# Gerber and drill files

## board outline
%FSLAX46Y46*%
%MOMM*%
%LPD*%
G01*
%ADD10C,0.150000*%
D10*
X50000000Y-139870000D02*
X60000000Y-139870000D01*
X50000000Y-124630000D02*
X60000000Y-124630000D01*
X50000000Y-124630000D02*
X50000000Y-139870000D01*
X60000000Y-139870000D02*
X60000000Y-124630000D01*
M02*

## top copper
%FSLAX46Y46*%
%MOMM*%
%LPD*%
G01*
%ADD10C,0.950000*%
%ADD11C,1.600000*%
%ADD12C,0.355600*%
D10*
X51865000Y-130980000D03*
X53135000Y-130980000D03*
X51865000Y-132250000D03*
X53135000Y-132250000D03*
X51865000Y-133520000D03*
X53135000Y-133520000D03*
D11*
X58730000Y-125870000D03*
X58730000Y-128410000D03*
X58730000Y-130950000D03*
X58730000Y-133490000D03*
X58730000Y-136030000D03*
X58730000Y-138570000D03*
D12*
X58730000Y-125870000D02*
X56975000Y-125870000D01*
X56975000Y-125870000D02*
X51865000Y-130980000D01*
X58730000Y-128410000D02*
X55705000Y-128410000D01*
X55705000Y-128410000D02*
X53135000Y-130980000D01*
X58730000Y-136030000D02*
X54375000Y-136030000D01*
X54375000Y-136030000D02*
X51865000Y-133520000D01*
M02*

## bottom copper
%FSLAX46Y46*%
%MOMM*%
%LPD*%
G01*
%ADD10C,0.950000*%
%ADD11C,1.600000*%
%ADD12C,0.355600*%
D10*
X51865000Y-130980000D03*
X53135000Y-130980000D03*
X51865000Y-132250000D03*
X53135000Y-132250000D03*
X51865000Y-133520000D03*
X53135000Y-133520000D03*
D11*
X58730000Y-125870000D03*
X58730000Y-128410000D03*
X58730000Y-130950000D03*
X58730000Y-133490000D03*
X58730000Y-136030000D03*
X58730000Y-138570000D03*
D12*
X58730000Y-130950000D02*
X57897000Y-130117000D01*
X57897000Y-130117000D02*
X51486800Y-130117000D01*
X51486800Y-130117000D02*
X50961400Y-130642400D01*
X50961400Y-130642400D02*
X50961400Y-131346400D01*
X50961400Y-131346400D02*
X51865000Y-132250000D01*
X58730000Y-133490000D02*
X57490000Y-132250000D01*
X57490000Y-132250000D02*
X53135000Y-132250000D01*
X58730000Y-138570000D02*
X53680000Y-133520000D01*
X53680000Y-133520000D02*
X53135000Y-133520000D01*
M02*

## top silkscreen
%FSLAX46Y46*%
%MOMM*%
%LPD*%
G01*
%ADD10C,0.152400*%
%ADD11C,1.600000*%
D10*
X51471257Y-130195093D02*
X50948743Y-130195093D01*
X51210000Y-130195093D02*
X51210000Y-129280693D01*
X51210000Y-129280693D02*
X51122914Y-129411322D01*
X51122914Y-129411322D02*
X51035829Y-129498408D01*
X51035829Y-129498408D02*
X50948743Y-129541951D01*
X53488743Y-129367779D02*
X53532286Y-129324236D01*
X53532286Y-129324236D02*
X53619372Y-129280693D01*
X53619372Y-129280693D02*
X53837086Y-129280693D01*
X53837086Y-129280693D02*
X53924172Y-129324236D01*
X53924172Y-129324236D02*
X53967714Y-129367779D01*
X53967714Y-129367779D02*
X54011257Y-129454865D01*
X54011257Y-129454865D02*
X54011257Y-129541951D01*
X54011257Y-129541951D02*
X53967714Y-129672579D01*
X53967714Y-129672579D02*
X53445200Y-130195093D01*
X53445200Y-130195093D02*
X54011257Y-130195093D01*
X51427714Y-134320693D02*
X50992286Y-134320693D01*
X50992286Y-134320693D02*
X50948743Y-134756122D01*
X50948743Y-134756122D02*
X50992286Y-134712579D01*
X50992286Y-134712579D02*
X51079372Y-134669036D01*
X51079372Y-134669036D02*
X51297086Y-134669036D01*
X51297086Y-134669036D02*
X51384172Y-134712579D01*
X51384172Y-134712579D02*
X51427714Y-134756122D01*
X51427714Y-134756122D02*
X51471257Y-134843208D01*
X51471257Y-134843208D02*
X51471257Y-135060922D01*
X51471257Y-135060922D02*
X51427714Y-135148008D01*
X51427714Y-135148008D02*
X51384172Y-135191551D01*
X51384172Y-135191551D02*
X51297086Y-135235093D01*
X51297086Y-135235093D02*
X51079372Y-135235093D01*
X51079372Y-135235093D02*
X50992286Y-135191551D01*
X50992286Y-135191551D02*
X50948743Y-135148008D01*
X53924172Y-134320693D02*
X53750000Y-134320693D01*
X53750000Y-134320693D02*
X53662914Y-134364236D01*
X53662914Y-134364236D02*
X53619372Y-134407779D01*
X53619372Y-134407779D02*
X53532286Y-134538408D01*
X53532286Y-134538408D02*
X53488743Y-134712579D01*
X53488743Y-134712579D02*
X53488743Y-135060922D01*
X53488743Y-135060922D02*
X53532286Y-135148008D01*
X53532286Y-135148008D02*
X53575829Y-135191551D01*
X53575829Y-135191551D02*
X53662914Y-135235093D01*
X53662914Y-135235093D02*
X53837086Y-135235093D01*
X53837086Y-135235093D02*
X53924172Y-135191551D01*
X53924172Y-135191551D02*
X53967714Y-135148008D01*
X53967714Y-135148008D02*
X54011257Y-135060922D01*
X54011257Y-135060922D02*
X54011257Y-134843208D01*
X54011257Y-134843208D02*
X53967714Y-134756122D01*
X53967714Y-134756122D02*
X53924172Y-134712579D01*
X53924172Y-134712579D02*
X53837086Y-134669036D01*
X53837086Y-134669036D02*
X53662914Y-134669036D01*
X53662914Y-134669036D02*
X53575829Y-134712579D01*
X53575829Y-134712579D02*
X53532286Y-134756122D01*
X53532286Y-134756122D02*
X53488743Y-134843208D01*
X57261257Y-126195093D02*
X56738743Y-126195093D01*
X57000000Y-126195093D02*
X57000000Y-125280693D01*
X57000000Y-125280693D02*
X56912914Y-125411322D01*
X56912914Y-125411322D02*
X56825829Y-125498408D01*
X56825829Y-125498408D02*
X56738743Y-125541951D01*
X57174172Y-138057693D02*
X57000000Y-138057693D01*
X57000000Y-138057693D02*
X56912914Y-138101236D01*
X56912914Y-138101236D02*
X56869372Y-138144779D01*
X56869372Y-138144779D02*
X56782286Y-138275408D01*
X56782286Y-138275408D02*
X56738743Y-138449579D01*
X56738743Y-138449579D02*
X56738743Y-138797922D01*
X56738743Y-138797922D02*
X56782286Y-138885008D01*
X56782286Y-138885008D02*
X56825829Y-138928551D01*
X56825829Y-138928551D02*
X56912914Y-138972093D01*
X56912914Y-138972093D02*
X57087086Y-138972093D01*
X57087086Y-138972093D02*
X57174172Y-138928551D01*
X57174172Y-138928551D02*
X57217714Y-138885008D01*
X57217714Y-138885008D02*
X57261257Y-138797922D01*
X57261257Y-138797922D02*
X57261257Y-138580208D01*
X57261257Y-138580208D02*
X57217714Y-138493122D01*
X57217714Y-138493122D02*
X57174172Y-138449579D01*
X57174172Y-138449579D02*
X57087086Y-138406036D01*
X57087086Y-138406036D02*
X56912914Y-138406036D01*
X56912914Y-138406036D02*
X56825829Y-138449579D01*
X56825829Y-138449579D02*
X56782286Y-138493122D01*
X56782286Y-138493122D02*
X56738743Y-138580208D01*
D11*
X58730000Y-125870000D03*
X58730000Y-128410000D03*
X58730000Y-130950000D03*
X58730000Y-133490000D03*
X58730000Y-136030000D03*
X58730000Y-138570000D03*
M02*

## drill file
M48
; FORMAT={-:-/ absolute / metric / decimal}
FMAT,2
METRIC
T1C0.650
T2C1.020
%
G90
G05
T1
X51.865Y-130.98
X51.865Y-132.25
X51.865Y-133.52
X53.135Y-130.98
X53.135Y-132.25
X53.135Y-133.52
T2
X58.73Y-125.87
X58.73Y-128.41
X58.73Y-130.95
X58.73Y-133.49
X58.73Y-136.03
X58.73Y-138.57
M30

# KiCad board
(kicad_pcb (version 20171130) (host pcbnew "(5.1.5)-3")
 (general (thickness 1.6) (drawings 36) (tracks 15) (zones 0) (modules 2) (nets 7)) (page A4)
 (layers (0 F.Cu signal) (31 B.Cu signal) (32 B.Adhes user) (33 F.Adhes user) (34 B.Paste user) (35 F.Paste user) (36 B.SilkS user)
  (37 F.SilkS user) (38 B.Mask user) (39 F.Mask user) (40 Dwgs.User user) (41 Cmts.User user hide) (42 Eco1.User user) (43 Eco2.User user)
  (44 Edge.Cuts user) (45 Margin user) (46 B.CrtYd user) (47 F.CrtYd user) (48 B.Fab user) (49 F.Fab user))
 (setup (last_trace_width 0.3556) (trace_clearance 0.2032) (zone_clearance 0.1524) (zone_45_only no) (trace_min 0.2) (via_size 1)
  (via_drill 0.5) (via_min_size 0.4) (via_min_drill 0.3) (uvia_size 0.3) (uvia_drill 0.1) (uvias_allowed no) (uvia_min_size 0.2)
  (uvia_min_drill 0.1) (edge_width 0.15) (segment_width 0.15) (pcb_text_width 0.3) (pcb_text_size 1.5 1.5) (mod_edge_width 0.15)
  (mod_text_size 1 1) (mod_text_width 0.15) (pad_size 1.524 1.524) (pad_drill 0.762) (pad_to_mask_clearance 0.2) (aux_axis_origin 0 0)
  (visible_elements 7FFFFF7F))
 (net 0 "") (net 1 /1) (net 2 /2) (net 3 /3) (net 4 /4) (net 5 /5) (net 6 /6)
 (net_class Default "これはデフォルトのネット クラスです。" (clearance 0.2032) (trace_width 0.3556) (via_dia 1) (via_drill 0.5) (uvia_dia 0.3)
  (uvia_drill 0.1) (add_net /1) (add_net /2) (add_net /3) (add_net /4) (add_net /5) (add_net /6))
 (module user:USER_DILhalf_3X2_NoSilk (layer F.Cu) (at 52.5 132.25)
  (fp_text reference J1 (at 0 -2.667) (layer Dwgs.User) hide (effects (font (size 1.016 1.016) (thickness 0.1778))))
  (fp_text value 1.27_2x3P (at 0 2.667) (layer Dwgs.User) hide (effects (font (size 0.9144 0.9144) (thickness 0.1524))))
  (pad 1 thru_hole circle (at -0.635 -1.27) (size 0.95 0.95) (drill 0.65) (layers *.Cu *.Mask) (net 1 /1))
  (pad 2 thru_hole circle (at 0.635 -1.27) (size 0.95 0.95) (drill 0.65) (layers *.Cu *.Mask) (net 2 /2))
  (pad 3 thru_hole circle (at -0.635 0) (size 0.95 0.95) (drill 0.65) (layers *.Cu *.Mask) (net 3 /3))
  (pad 4 thru_hole circle (at 0.635 0) (size 0.95 0.95) (drill 0.65) (layers *.Cu *.Mask) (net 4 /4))
  (pad 5 thru_hole circle (at -0.635 1.27) (size 0.95 0.95) (drill 0.65) (layers *.Cu *.Mask) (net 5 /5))
  (pad 6 thru_hole circle (at 0.635 1.27) (size 0.95 0.95) (drill 0.65) (layers *.Cu *.Mask) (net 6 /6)))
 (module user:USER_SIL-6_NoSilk (layer F.Cu) (at 58.73 132.22 270)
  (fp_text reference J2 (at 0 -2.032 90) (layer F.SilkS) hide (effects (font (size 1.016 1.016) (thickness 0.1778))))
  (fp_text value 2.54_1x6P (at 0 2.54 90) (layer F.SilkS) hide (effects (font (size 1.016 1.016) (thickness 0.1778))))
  (pad 1 thru_hole circle (at -6.35 0 270) (size 1.6 1.6) (drill 1.02) (layers *.Cu *.Mask F.SilkS) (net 1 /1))
  (pad 2 thru_hole circle (at -3.81 0 270) (size 1.6 1.6) (drill 1.02) (layers *.Cu *.Mask F.SilkS) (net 2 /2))
  (pad 3 thru_hole circle (at -1.27 0 270) (size 1.6 1.6) (drill 1.02) (layers *.Cu *.Mask F.SilkS) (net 3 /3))
  (pad 4 thru_hole circle (at 1.27 0 270) (size 1.6 1.6) (drill 1.02) (layers *.Cu *.Mask F.SilkS) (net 4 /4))
  (pad 5 thru_hole circle (at 3.81 0 270) (size 1.6 1.6) (drill 1.02) (layers *.Cu *.Mask F.SilkS) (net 5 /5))
  (pad 6 thru_hole circle (at 6.35 0 270) (size 1.6 1.6) (drill 1.02) (layers *.Cu *.Mask F.SilkS) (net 6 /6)))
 (gr_line (start 50 139.87) (end 60 139.87) (angle 90) (layer Edge.Cuts) (width 0.15))
 (gr_line (start 50 124.63) (end 60 124.63) (angle 90) (layer Edge.Cuts) (width 0.15))
 (gr_line (start 50 124.63) (end 50 139.87) (angle 90) (layer Edge.Cuts) (width 0.15))
 (gr_line (start 60 139.87) (end 60 124.63) (angle 90) (layer Edge.Cuts) (width 0.15))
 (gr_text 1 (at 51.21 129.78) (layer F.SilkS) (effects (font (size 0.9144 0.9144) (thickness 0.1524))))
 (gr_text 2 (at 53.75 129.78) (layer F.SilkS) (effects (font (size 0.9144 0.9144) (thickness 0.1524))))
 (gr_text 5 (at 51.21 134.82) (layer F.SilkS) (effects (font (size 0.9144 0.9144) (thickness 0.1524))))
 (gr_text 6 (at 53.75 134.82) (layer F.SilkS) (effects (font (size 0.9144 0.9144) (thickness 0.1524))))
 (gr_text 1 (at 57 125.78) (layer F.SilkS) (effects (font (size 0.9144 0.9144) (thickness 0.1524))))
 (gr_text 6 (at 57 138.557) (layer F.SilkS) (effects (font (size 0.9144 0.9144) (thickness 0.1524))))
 (segment (start 58.73 125.87) (end 56.975 125.87) (width 0.3556) (layer F.Cu) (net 1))
 (segment (start 56.975 125.87) (end 51.865 130.98) (width 0.3556) (layer F.Cu) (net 1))
 (segment (start 58.73 128.41) (end 55.705 128.41) (width 0.3556) (layer F.Cu) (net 2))
 (segment (start 55.705 128.41) (end 53.135 130.98) (width 0.3556) (layer F.Cu) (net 2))
 (segment (start 58.73 130.95) (end 57.897 130.117) (width 0.3556) (layer B.Cu) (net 3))
 (segment (start 57.897 130.117) (end 51.4868 130.117) (width 0.3556) (layer B.Cu) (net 3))
 (segment (start 51.4868 130.117) (end 50.9614 130.6424) (width 0.3556) (layer B.Cu) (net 3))
 (segment (start 50.9614 130.6424) (end 50.9614 131.3464) (width 0.3556) (layer B.Cu) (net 3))
 (segment (start 50.9614 131.3464) (end 51.865 132.25) (width 0.3556) (layer B.Cu) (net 3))
 (segment (start 58.73 133.49) (end 57.49 132.25) (width 0.3556) (layer B.Cu) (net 4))
 (segment (start 57.49 132.25) (end 53.135 132.25) (width 0.3556) (layer B.Cu) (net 4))
 (segment (start 58.73 136.03) (end 54.375 136.03) (width 0.3556) (layer F.Cu) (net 5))
 (segment (start 54.375 136.03) (end 51.865 133.52) (width 0.3556) (layer F.Cu) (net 5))
 (segment (start 58.73 138.57) (end 53.68 133.52) (width 0.3556) (layer B.Cu) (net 6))
 (segment (start 53.68 133.52) (end 53.135 133.52) (width 0.3556) (layer B.Cu) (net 6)))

